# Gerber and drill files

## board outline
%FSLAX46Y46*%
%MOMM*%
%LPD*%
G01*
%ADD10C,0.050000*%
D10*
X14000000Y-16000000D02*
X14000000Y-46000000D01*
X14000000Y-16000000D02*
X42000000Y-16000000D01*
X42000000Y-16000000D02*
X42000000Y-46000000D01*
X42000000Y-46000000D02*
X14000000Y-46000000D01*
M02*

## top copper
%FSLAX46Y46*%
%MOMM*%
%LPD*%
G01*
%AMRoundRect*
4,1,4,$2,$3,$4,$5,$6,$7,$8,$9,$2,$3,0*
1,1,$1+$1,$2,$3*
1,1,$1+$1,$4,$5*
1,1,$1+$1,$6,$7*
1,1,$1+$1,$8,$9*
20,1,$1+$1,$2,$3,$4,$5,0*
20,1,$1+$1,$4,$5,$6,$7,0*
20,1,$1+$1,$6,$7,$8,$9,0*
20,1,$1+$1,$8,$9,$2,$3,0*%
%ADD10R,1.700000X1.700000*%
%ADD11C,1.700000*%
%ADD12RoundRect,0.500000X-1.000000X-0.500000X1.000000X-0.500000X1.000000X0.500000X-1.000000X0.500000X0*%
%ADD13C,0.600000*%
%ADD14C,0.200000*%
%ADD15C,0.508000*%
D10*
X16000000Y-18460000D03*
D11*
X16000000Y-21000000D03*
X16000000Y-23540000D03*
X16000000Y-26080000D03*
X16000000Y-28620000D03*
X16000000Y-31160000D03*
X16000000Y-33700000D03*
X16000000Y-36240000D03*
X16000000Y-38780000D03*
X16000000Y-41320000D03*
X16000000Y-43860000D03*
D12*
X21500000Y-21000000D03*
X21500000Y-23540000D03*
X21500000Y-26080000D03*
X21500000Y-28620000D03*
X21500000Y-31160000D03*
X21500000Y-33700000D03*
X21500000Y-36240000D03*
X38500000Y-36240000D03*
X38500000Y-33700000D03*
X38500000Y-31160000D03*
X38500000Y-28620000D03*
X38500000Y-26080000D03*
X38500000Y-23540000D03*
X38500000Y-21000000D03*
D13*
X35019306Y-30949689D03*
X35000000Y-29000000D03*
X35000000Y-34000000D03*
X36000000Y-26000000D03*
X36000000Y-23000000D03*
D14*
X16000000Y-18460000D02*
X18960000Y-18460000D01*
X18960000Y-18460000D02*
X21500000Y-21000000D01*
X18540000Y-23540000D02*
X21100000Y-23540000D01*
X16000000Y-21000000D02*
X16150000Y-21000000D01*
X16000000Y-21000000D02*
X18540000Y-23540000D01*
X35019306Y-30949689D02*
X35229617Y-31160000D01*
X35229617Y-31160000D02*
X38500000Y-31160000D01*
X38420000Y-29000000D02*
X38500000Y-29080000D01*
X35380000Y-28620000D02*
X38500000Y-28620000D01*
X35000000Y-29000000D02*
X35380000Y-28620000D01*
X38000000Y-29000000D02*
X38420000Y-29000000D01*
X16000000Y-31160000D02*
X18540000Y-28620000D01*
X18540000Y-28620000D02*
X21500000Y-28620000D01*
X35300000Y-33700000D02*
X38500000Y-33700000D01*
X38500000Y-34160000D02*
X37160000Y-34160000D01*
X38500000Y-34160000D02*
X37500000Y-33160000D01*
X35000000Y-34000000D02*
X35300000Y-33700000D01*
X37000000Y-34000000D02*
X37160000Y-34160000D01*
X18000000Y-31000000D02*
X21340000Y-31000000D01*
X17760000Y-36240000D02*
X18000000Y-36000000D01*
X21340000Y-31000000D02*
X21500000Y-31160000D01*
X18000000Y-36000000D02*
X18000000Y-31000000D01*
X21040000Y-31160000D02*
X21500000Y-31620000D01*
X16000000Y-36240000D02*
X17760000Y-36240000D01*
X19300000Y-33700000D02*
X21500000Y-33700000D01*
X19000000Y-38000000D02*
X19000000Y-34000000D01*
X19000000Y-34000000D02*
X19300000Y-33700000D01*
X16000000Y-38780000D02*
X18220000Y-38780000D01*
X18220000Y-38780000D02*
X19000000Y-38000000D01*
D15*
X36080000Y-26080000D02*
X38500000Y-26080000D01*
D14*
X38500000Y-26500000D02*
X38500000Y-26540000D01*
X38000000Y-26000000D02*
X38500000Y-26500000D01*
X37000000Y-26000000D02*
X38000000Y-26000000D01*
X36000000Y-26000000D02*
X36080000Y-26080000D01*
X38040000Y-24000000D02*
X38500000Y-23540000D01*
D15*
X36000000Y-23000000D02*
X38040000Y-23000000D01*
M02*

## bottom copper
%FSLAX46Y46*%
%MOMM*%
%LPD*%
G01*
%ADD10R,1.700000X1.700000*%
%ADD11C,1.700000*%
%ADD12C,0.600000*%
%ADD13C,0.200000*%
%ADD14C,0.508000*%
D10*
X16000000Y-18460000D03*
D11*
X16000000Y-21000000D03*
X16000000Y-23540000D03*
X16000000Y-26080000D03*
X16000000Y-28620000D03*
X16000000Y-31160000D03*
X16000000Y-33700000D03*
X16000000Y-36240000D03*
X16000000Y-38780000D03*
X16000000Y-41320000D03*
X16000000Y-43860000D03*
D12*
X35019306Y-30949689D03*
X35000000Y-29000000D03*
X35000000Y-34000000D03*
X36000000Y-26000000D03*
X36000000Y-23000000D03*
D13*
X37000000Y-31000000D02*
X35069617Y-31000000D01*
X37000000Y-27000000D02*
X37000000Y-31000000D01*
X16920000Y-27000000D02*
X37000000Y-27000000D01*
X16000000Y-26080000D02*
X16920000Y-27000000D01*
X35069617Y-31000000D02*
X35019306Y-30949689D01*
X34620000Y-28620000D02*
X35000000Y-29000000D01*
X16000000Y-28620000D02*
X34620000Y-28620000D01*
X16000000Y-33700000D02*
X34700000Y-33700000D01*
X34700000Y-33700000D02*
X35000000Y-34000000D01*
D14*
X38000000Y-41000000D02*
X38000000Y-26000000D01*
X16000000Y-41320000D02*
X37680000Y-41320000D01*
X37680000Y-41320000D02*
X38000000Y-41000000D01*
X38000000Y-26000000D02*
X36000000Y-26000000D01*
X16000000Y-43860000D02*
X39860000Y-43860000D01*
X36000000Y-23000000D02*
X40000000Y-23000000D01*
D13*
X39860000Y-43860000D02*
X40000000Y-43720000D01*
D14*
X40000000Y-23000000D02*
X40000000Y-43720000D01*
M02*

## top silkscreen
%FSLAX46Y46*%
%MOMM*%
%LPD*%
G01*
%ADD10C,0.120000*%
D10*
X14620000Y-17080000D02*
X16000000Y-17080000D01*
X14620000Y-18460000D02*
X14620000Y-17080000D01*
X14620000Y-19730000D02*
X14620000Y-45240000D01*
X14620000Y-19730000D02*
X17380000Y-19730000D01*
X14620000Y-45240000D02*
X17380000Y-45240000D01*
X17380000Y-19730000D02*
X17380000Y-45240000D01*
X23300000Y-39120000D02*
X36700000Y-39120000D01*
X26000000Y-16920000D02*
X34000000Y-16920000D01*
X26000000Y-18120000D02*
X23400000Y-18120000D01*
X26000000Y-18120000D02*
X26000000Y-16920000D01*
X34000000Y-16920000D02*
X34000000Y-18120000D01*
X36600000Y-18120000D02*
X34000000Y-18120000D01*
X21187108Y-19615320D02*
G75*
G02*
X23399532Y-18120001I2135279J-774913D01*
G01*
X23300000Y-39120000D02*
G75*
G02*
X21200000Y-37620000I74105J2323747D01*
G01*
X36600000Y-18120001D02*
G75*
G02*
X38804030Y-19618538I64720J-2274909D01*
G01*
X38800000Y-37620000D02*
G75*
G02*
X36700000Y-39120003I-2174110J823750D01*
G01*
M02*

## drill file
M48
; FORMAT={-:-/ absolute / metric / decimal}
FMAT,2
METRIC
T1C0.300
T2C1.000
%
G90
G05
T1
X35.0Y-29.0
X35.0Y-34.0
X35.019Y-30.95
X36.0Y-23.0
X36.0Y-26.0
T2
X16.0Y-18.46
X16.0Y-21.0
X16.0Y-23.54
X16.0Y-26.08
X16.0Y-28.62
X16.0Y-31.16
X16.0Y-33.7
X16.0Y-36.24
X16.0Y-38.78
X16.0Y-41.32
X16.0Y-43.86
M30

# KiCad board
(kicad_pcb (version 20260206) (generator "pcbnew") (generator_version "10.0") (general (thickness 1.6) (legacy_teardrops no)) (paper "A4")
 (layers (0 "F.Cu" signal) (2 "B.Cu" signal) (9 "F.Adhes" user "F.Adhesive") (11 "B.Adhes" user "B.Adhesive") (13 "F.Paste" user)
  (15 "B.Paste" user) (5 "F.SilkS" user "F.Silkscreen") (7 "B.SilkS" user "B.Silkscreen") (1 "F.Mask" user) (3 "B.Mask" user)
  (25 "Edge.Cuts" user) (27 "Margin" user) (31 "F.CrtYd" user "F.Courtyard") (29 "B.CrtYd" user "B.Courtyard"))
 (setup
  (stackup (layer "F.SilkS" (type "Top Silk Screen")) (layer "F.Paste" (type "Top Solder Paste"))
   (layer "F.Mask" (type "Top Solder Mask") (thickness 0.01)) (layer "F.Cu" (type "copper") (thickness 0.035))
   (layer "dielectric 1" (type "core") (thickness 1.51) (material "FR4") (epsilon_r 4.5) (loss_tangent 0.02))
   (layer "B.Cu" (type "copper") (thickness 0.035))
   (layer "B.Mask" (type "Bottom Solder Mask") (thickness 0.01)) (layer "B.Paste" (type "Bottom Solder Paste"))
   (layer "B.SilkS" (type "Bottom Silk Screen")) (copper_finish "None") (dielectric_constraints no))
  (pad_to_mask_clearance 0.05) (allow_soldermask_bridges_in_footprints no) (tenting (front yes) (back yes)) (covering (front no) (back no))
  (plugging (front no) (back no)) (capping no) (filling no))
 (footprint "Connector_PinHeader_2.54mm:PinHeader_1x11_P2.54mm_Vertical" (layer "F.Cu") (at 16 18.46)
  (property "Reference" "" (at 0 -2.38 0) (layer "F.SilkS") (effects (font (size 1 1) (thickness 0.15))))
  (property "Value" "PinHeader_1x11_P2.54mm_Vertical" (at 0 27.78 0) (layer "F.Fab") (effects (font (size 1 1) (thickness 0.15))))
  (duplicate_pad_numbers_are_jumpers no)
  (fp_line (start -1.38 -1.38) (end 0 -1.38) (stroke (width 0.12) (type solid)) (layer "F.SilkS"))
  (fp_line (start -1.38 0) (end -1.38 -1.38) (stroke (width 0.12) (type solid)) (layer "F.SilkS"))
  (fp_line (start -1.38 1.27) (end -1.38 26.78) (stroke (width 0.12) (type solid)) (layer "F.SilkS"))
  (fp_line (start -1.38 1.27) (end 1.38 1.27) (stroke (width 0.12) (type solid)) (layer "F.SilkS"))
  (fp_line (start -1.38 26.78) (end 1.38 26.78) (stroke (width 0.12) (type solid)) (layer "F.SilkS"))
  (fp_line (start 1.38 1.27) (end 1.38 26.78) (stroke (width 0.12) (type solid)) (layer "F.SilkS"))
  (pad "1" thru_hole rect (at 0 0) (size 1.7 1.7) (drill 1) (layers "*.Cu" "*.Mask") (remove_unused_layers no) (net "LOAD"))
  (pad "2" thru_hole circle (at 0 2.54) (size 1.7 1.7) (drill 1) (layers "*.Cu" "*.Mask") (remove_unused_layers no) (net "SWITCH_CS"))
  (pad "3" thru_hole circle (at 0 5.08) (size 1.7 1.7) (drill 1) (layers "*.Cu" "*.Mask") (remove_unused_layers no))
  (pad "4" thru_hole circle (at 0 7.62) (size 1.7 1.7) (drill 1) (layers "*.Cu" "*.Mask") (remove_unused_layers no) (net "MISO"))
  (pad "5" thru_hole circle (at 0 10.16) (size 1.7 1.7) (drill 1) (layers "*.Cu" "*.Mask") (remove_unused_layers no) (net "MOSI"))
  (pad "6" thru_hole circle (at 0 12.7) (size 1.7 1.7) (drill 1) (layers "*.Cu" "*.Mask") (remove_unused_layers no) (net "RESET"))
  (pad "7" thru_hole circle (at 0 15.24) (size 1.7 1.7) (drill 1) (layers "*.Cu" "*.Mask") (remove_unused_layers no) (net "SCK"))
  (pad "8" thru_hole circle (at 0 17.78) (size 1.7 1.7) (drill 1) (layers "*.Cu" "*.Mask") (remove_unused_layers no) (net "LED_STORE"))
  (pad "9" thru_hole circle (at 0 20.32) (size 1.7 1.7) (drill 1) (layers "*.Cu" "*.Mask") (remove_unused_layers no) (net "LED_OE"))
  (pad "10" thru_hole circle (at 0 22.86) (size 1.7 1.7) (drill 1) (layers "*.Cu" "*.Mask") (remove_unused_layers no) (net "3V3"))
  (pad "11" thru_hole circle (at 0 25.4) (size 1.7 1.7) (drill 1) (layers "*.Cu" "*.Mask") (remove_unused_layers no) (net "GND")))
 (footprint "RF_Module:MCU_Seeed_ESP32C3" (layer "F.Cu") (at 30 28.62)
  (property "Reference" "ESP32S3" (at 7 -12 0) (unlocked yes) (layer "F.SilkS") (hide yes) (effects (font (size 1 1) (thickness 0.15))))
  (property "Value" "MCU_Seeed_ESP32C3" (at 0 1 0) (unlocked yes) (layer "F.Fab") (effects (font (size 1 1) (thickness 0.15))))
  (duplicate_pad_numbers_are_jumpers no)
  (fp_line (start -6.7 10.5) (end 6.7 10.5) (stroke (width 0.12) (type default)) (layer "F.SilkS"))
  (fp_line (start -4 -11.7) (end 4 -11.7) (stroke (width 0.12) (type default)) (layer "F.SilkS"))
  (fp_line (start -4 -10.5) (end -6.6 -10.5) (stroke (width 0.12) (type default)) (layer "F.SilkS"))
  (fp_line (start -4 -10.5) (end -4 -11.7) (stroke (width 0.12) (type default)) (layer "F.SilkS"))
  (fp_line (start 4 -11.7) (end 4 -10.5) (stroke (width 0.12) (type default)) (layer "F.SilkS"))
  (fp_line (start 6.6 -10.5) (end 4 -10.5) (stroke (width 0.12) (type default)) (layer "F.SilkS"))
  (fp_arc (start -8.812892 -9.00468) (mid -7.949609 -10.111769) (end -6.600468 -10.499999) (stroke (width 0.12) (type default))
   (layer "F.SilkS"))
  (fp_arc (start -6.7 10.5) (mid -7.977232 10.068125) (end -8.8 9) (stroke (width 0.12) (type default)) (layer "F.SilkS"))
  (fp_arc (start 6.6 -10.499999) (mid 7.944325 -10.107116) (end 8.804034 -9.001464) (stroke (width 0.12) (type default)) (layer "F.SilkS"))
  (fp_arc (start 8.8 9) (mid 7.977232 10.068125) (end 6.7 10.5) (stroke (width 0.12) (type default)) (layer "F.SilkS"))
  (pad "1" smd roundrect (at -8.5 -7.62) (size 3 2) (layers "F.Cu" "F.Mask" "F.Paste") (roundrect_rratio 0.25) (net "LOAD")
   (thermal_bridge_angle 45))
  (pad "2" smd roundrect (at -8.5 -5.08) (size 3 2) (layers "F.Cu" "F.Mask" "F.Paste") (roundrect_rratio 0.25) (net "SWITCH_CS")
   (thermal_bridge_angle 45))
  (pad "3" smd roundrect (at -8.5 -2.54) (size 3 2) (layers "F.Cu" "F.Mask" "F.Paste") (roundrect_rratio 0.25) (thermal_bridge_angle 45))
  (pad "4" smd roundrect (at -8.5 0) (size 3 2) (layers "F.Cu" "F.Mask" "F.Paste") (roundrect_rratio 0.25) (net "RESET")
   (thermal_bridge_angle 45))
  (pad "5" smd roundrect (at -8.5 2.54) (size 3 2) (layers "F.Cu" "F.Mask" "F.Paste") (roundrect_rratio 0.25) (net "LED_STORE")
   (thermal_bridge_angle 45))
  (pad "6" smd roundrect (at -8.5 5.08) (size 3 2) (layers "F.Cu" "F.Mask" "F.Paste") (roundrect_rratio 0.25) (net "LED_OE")
   (thermal_bridge_angle 45))
  (pad "7" smd roundrect (at -8.5 7.62) (size 3 2) (layers "F.Cu" "F.Mask" "F.Paste") (roundrect_rratio 0.25) (thermal_bridge_angle 45))
  (pad "8" smd roundrect (at 8.5 7.62) (size 3 2) (layers "F.Cu" "F.Mask" "F.Paste") (roundrect_rratio 0.25) (thermal_bridge_angle 45))
  (pad "9" smd roundrect (at 8.5 5.08) (size 3 2) (layers "F.Cu" "F.Mask" "F.Paste") (roundrect_rratio 0.25) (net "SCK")
   (thermal_bridge_angle 45))
  (pad "10" smd roundrect (at 8.5 2.54) (size 3 2) (layers "F.Cu" "F.Mask" "F.Paste") (roundrect_rratio 0.25) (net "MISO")
   (thermal_bridge_angle 45))
  (pad "11" smd roundrect (at 8.5 0) (size 3 2) (layers "F.Cu" "F.Mask" "F.Paste") (roundrect_rratio 0.25) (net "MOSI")
   (thermal_bridge_angle 45))
  (pad "12" smd roundrect (at 8.5 -2.54) (size 3 2) (layers "F.Cu" "F.Mask" "F.Paste") (roundrect_rratio 0.25) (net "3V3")
   (thermal_bridge_angle 45))
  (pad "13" smd roundrect (at 8.5 -5.08) (size 3 2) (layers "F.Cu" "F.Mask" "F.Paste") (roundrect_rratio 0.25) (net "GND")
   (thermal_bridge_angle 45))
  (pad "14" smd roundrect (at 8.5 -7.62) (size 3 2) (layers "F.Cu" "F.Mask" "F.Paste") (roundrect_rratio 0.25) (thermal_bridge_angle 45)))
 (gr_line (start 14 16) (end 14 46) (stroke (width 0.05) (type default)) (layer "Edge.Cuts"))
 (gr_line (start 14 16) (end 42 16) (stroke (width 0.05) (type default)) (layer "Edge.Cuts"))
 (gr_line (start 42 16) (end 42 46) (stroke (width 0.05) (type default)) (layer "Edge.Cuts"))
 (gr_line (start 42 46) (end 14 46) (stroke (width 0.05) (type default)) (layer "Edge.Cuts"))
 (segment (start 16 18.46) (end 18.96 18.46) (width 0.2) (layer "F.Cu") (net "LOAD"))
 (segment (start 18.96 18.46) (end 21.5 21) (width 0.2) (layer "F.Cu") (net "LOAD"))
 (segment (start 18.54 23.54) (end 21.1 23.54) (width 0.2) (layer "F.Cu") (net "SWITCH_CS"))
 (segment (start 16 21) (end 16.15 21) (width 0.2) (layer "F.Cu") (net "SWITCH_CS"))
 (segment (start 16 21) (end 18.54 23.54) (width 0.2) (layer "F.Cu") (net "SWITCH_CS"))
 (segment (start 35.019306 30.949689) (end 35.229617 31.16) (width 0.2) (layer "F.Cu") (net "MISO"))
 (segment (start 35.229617 31.16) (end 38.5 31.16) (width 0.2) (layer "F.Cu") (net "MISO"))
 (via (at 35.019306 30.949689) (size 0.6) (drill 0.3) (layers "F.Cu" "B.Cu") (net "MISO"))
 (segment (start 37 31) (end 35.069617 31) (width 0.2) (layer "B.Cu") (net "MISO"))
 (segment (start 37 27) (end 37 31) (width 0.2) (layer "B.Cu") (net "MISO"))
 (segment (start 16.92 27) (end 37 27) (width 0.2) (layer "B.Cu") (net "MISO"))
 (segment (start 16 26.08) (end 16.92 27) (width 0.2) (layer "B.Cu") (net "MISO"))
 (segment (start 35.069617 31) (end 35.019306 30.949689) (width 0.2) (layer "B.Cu") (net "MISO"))
 (segment (start 38.42 29) (end 38.5 29.08) (width 0.2) (layer "F.Cu") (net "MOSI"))
 (segment (start 35.38 28.62) (end 38.5 28.62) (width 0.2) (layer "F.Cu") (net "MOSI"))
 (segment (start 35 29) (end 35.38 28.62) (width 0.2) (layer "F.Cu") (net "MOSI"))
 (segment (start 38 29) (end 38.42 29) (width 0.2) (layer "F.Cu") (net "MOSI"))
 (via (at 35 29) (size 0.6) (drill 0.3) (layers "F.Cu" "B.Cu") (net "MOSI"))
 (segment (start 34.62 28.62) (end 35 29) (width 0.2) (layer "B.Cu") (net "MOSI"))
 (segment (start 16 28.62) (end 34.62 28.62) (width 0.2) (layer "B.Cu") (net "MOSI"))
 (segment (start 16 31.16) (end 18.54 28.62) (width 0.2) (layer "F.Cu") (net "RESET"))
 (segment (start 18.54 28.62) (end 21.5 28.62) (width 0.2) (layer "F.Cu") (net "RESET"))
 (segment (start 35.3 33.7) (end 38.5 33.7) (width 0.2) (layer "F.Cu") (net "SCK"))
 (segment (start 38.5 34.16) (end 37.16 34.16) (width 0.2) (layer "F.Cu") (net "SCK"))
 (segment (start 38.5 34.16) (end 37.5 33.16) (width 0.2) (layer "F.Cu") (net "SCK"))
 (segment (start 35 34) (end 35.3 33.7) (width 0.2) (layer "F.Cu") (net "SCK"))
 (segment (start 37 34) (end 37.16 34.16) (width 0.2) (layer "F.Cu") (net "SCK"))
 (via (at 35 34) (size 0.6) (drill 0.3) (layers "F.Cu" "B.Cu") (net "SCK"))
 (segment (start 16 33.7) (end 34.7 33.7) (width 0.2) (layer "B.Cu") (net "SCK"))
 (segment (start 34.7 33.7) (end 35 34) (width 0.2) (layer "B.Cu") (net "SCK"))
 (segment (start 18 31) (end 21.34 31) (width 0.2) (layer "F.Cu") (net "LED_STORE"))
 (segment (start 17.76 36.24) (end 18 36) (width 0.2) (layer "F.Cu") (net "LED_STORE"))
 (segment (start 21.34 31) (end 21.5 31.16) (width 0.2) (layer "F.Cu") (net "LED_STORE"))
 (segment (start 18 36) (end 18 31) (width 0.2) (layer "F.Cu") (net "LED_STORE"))
 (segment (start 21.04 31.16) (end 21.5 31.62) (width 0.2) (layer "F.Cu") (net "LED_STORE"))
 (segment (start 16 36.24) (end 17.76 36.24) (width 0.2) (layer "F.Cu") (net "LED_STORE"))
 (segment (start 19.3 33.7) (end 21.5 33.7) (width 0.2) (layer "F.Cu") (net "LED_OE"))
 (segment (start 19 38) (end 19 34) (width 0.2) (layer "F.Cu") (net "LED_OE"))
 (segment (start 19 34) (end 19.3 33.7) (width 0.2) (layer "F.Cu") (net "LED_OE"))
 (segment (start 16 38.78) (end 18.22 38.78) (width 0.2) (layer "F.Cu") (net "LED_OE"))
 (segment (start 18.22 38.78) (end 19 38) (width 0.2) (layer "F.Cu") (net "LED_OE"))
 (segment (start 36.08 26.08) (end 38.5 26.08) (width 0.508) (layer "F.Cu") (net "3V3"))
 (segment (start 38.5 26.5) (end 38.5 26.54) (width 0.2) (layer "F.Cu") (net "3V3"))
 (segment (start 38 26) (end 38.5 26.5) (width 0.2) (layer "F.Cu") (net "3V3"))
 (segment (start 37 26) (end 38 26) (width 0.2) (layer "F.Cu") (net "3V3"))
 (segment (start 36 26) (end 36.08 26.08) (width 0.2) (layer "F.Cu") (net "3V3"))
 (via (at 36 26) (size 0.6) (drill 0.3) (layers "F.Cu" "B.Cu") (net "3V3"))
 (segment (start 38 41) (end 38 26) (width 0.508) (layer "B.Cu") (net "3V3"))
 (segment (start 16 41.32) (end 37.68 41.32) (width 0.508) (layer "B.Cu") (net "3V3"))
 (segment (start 37.68 41.32) (end 38 41) (width 0.508) (layer "B.Cu") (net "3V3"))
 (segment (start 38 26) (end 36 26) (width 0.508) (layer "B.Cu") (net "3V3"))
 (segment (start 38.04 24) (end 38.5 23.54) (width 0.2) (layer "F.Cu") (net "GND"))
 (segment (start 36 23) (end 38.04 23) (width 0.508) (layer "F.Cu") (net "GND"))
 (via (at 36 23) (size 0.6) (drill 0.3) (layers "F.Cu" "B.Cu") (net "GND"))
 (segment (start 16 43.86) (end 39.86 43.86) (width 0.508) (layer "B.Cu") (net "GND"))
 (segment (start 36 23) (end 40 23) (width 0.508) (layer "B.Cu") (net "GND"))
 (segment (start 39.86 43.86) (end 40 43.72) (width 0.2) (layer "B.Cu") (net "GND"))
 (segment (start 40 23) (end 40 43.72) (width 0.508) (layer "B.Cu") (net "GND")))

